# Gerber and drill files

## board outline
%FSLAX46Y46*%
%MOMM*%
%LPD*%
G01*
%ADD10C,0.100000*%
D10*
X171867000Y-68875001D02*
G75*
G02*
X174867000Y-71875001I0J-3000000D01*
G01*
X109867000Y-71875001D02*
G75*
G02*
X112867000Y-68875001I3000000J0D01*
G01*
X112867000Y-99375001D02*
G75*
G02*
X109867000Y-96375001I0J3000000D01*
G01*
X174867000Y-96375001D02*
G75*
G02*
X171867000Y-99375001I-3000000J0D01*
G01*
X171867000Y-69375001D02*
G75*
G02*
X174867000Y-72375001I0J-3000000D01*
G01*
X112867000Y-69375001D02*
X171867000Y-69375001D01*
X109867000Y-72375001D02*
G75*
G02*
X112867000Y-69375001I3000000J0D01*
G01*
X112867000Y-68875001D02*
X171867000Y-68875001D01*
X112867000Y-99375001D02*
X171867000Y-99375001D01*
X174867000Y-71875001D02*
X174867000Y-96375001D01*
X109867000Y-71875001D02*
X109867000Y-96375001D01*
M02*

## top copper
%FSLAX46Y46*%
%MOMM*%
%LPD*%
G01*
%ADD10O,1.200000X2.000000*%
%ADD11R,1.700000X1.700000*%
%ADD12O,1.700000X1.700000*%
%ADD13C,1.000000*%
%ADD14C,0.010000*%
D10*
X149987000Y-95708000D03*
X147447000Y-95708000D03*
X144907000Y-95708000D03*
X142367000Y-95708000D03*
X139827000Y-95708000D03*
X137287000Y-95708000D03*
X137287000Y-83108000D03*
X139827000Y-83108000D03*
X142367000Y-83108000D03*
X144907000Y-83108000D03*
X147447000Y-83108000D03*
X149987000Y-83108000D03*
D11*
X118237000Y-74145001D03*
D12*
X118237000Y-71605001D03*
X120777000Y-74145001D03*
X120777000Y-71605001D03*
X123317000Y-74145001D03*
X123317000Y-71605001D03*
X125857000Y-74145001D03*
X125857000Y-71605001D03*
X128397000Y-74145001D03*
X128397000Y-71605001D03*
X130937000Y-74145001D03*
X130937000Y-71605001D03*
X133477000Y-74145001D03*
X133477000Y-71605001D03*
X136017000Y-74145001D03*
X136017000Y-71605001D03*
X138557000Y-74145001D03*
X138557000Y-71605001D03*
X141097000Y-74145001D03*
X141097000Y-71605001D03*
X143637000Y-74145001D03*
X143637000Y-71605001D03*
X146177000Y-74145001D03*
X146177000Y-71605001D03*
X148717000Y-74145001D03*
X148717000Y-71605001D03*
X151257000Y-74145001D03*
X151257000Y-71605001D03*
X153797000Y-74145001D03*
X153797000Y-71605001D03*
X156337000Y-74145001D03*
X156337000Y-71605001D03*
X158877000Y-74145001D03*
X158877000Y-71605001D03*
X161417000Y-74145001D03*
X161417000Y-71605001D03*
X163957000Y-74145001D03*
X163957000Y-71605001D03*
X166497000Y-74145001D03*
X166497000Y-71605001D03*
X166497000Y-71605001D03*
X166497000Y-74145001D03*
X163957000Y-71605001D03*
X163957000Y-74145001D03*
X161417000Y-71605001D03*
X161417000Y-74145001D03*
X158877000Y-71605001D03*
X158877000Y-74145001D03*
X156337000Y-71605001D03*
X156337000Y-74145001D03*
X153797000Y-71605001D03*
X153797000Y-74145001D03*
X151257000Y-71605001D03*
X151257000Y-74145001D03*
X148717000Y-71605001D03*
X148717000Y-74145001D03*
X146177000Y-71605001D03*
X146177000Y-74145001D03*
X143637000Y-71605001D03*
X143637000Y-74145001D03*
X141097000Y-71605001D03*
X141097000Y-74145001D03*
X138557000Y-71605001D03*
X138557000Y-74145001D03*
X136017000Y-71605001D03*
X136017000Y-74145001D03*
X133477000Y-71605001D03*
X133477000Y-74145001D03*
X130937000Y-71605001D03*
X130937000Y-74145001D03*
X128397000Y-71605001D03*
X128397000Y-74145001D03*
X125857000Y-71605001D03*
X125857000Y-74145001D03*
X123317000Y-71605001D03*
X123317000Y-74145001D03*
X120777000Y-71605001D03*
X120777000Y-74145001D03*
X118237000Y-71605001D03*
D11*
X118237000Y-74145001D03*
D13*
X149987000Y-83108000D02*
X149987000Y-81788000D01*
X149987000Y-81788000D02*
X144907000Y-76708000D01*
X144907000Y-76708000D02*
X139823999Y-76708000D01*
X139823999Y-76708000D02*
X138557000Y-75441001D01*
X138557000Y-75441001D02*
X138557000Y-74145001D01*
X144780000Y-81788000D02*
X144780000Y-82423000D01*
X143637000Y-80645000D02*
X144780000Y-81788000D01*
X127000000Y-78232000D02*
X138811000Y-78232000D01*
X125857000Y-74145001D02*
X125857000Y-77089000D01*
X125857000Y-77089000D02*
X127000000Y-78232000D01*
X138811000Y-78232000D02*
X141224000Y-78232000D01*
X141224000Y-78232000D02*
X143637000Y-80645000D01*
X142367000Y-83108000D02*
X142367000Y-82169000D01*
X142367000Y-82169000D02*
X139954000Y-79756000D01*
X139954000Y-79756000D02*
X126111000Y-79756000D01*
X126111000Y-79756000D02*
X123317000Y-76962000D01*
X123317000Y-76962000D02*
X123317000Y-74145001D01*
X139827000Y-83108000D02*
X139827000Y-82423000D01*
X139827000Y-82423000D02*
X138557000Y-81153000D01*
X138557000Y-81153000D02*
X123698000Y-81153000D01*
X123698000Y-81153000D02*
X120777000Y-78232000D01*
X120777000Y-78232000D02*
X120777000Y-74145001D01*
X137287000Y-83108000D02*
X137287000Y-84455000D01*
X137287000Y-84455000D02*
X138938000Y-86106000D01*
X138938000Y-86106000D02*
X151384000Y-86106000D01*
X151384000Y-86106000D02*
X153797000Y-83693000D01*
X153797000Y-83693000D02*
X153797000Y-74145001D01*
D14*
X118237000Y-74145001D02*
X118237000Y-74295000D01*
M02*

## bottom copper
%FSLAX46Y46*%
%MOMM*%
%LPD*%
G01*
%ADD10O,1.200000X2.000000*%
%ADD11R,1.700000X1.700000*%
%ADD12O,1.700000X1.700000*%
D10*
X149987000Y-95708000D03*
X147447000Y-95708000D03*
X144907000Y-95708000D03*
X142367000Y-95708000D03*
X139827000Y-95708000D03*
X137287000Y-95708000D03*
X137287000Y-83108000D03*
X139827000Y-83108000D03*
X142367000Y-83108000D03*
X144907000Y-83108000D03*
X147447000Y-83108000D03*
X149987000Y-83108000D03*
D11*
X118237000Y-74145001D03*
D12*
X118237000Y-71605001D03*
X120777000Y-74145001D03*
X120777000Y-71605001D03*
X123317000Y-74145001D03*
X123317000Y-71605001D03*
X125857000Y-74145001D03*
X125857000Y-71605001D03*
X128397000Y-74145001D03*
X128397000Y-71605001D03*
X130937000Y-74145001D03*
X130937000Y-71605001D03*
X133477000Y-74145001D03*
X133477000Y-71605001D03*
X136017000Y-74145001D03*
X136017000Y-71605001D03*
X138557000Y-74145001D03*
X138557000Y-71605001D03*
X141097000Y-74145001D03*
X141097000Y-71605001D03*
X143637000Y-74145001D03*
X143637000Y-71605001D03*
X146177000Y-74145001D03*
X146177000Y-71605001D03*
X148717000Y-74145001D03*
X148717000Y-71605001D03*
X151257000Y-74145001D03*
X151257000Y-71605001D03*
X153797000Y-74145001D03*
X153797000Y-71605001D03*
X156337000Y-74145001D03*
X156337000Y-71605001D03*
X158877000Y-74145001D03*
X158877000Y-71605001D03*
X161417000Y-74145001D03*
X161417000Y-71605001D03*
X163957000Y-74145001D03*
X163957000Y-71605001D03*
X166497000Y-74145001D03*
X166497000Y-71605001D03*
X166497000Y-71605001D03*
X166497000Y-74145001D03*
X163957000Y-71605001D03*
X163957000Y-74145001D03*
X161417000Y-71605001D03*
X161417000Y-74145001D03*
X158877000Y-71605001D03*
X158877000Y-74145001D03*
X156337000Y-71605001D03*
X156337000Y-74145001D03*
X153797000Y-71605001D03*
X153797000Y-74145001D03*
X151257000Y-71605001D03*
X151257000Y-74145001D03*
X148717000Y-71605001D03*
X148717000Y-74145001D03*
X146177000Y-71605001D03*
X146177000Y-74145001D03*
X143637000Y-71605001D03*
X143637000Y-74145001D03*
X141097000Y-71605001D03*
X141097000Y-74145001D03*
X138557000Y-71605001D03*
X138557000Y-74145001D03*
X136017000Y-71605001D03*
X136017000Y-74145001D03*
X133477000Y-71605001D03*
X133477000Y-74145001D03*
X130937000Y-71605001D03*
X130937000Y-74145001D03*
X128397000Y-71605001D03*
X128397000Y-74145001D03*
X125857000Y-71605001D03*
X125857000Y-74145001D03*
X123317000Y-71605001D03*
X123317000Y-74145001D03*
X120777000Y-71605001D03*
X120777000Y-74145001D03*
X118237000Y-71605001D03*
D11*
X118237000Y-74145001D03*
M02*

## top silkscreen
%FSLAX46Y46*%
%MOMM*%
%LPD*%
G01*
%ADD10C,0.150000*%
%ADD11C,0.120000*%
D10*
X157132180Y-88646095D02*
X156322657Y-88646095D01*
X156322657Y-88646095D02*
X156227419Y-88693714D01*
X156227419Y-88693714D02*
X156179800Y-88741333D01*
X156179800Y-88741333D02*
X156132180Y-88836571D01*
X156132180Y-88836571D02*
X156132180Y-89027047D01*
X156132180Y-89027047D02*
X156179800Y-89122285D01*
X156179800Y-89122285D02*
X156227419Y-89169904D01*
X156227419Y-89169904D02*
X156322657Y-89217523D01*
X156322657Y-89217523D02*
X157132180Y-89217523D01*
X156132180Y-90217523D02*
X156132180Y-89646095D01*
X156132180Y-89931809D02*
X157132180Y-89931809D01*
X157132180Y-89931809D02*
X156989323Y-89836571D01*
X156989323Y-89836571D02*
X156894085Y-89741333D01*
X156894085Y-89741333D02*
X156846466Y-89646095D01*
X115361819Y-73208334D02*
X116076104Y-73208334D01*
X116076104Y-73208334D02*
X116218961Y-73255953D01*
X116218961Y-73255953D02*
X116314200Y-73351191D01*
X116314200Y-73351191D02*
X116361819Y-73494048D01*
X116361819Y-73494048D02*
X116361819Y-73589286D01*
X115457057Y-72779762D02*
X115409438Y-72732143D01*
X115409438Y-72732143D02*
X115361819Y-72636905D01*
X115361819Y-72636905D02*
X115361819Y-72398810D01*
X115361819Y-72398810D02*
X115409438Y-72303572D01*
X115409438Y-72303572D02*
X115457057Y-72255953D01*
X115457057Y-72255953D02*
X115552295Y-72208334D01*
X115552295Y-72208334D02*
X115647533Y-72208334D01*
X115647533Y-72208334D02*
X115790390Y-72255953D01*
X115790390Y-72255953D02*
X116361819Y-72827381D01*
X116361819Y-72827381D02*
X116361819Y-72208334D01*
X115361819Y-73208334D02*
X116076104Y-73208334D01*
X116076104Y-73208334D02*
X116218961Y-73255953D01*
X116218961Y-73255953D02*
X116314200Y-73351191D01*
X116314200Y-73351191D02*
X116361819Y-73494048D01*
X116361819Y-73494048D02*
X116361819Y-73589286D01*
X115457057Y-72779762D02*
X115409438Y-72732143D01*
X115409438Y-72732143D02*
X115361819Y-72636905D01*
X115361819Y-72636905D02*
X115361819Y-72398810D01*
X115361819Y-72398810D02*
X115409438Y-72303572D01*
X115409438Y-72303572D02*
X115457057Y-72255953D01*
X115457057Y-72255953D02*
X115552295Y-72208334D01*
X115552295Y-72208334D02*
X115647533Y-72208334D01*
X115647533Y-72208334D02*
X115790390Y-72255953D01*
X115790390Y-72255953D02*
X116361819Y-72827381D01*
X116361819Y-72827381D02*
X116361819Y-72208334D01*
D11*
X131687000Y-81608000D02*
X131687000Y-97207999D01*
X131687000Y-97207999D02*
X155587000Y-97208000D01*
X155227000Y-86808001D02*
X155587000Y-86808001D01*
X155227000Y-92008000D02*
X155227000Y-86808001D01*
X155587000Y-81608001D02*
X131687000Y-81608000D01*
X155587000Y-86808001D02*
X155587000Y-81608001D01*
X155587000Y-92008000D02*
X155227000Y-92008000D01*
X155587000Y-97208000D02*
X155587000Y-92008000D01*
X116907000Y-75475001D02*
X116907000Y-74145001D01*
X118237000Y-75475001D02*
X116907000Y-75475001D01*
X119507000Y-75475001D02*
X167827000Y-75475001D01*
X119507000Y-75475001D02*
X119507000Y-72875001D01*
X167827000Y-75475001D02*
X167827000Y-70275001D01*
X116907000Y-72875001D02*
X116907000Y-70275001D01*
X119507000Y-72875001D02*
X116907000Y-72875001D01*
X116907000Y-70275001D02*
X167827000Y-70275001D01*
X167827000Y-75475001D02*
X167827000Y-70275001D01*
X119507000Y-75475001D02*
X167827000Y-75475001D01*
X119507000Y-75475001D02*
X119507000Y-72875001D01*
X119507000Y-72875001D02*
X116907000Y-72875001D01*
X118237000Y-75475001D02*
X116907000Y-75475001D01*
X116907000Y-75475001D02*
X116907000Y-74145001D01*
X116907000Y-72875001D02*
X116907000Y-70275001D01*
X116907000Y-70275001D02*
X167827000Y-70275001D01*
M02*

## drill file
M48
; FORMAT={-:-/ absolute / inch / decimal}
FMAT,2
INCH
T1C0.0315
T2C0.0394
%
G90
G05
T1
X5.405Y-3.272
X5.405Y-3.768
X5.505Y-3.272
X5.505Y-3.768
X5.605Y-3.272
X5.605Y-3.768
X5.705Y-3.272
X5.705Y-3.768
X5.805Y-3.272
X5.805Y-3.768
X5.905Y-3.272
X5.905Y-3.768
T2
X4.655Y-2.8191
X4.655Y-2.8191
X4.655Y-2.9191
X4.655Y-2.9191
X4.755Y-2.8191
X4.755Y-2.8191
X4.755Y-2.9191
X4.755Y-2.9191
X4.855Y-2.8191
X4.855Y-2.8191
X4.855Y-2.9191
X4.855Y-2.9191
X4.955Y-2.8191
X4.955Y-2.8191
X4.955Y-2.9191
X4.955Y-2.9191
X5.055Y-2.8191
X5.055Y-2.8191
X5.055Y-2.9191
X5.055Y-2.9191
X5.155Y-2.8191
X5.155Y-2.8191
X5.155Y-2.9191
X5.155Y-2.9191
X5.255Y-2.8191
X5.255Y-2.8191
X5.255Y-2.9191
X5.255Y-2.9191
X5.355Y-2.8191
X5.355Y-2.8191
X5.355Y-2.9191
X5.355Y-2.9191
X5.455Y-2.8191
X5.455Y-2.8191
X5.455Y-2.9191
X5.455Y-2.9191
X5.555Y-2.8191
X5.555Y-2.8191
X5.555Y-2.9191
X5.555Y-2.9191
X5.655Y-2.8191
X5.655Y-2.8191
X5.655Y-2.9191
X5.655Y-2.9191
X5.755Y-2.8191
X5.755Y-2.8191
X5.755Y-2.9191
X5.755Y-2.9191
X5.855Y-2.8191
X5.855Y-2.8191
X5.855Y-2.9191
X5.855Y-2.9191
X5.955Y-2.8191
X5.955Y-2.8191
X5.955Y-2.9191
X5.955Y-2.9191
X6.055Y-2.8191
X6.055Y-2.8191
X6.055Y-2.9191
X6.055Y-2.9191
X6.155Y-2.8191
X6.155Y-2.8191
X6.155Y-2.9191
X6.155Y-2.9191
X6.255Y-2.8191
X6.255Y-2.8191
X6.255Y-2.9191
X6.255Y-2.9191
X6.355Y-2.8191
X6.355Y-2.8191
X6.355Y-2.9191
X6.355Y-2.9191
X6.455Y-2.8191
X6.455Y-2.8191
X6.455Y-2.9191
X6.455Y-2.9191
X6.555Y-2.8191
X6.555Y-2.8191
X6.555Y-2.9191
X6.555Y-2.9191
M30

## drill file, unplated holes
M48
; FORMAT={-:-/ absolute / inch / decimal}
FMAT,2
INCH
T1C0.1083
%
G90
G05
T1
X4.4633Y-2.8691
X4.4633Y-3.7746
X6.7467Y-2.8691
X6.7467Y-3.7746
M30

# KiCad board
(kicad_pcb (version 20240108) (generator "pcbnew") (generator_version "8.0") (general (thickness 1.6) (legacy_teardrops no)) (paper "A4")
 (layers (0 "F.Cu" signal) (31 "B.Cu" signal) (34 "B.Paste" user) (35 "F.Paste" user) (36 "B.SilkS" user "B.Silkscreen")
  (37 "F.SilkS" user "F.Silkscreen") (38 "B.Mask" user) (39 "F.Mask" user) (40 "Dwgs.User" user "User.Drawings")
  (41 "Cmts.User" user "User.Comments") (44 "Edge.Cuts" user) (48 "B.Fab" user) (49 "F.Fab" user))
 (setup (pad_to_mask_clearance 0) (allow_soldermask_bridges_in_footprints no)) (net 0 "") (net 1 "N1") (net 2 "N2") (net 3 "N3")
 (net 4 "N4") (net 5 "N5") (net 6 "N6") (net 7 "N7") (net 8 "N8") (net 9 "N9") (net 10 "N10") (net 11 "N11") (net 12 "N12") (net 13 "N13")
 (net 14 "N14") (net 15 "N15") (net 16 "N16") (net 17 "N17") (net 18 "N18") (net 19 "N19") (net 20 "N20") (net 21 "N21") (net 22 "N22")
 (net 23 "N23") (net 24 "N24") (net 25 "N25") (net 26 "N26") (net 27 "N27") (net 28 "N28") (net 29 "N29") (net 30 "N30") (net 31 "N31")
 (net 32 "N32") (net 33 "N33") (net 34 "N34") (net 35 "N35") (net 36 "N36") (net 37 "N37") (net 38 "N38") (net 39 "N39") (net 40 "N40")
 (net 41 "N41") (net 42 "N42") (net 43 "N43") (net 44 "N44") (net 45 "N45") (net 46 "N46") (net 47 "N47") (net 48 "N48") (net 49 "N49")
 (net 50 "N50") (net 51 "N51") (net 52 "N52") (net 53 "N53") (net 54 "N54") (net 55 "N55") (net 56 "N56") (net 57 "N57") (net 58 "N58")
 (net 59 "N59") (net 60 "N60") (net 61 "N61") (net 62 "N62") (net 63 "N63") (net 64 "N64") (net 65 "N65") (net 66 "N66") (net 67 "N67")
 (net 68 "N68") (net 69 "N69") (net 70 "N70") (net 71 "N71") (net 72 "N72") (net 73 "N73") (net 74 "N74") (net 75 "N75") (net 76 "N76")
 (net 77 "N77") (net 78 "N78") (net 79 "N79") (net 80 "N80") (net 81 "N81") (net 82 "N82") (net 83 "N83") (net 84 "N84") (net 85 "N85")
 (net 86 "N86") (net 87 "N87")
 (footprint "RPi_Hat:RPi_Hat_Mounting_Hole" (layer "F.Cu") (at 171.367 72.875001)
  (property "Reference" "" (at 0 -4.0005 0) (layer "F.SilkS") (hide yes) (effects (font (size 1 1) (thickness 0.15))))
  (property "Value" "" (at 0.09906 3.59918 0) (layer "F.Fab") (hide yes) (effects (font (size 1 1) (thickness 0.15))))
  (pad "" np_thru_hole circle (at 0 0) (size 2.75 2.75) (drill 2.75) (layers "*.Cu" "*.Mask") (solder_mask_margin 1.725) (clearance 1.725)))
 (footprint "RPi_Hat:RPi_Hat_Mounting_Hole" (layer "F.Cu") (at 113.367 72.875001)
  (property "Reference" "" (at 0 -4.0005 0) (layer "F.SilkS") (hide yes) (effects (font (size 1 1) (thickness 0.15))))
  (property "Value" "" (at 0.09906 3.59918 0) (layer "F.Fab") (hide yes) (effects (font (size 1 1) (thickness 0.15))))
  (pad "" np_thru_hole circle (at 0 0) (size 2.75 2.75) (drill 2.75) (layers "*.Cu" "*.Mask") (solder_mask_margin 1.725) (clearance 1.725)))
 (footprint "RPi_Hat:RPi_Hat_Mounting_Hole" (layer "F.Cu") (at 171.367 95.875001)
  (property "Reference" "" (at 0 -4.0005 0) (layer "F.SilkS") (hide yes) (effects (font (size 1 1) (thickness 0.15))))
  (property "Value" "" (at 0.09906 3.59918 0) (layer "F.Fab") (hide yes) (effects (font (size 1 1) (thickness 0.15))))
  (pad "" np_thru_hole circle (at 0 0) (size 2.75 2.75) (drill 2.75) (layers "*.Cu" "*.Mask") (solder_mask_margin 1.725) (clearance 1.725)))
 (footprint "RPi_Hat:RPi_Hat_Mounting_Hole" (layer "F.Cu") (at 113.367 95.875001)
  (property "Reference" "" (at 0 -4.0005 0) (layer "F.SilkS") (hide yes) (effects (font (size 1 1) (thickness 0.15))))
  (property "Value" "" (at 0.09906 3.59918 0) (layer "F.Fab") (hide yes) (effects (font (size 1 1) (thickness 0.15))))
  (pad "" np_thru_hole circle (at 0 0) (size 2.75 2.75) (drill 2.75) (layers "*.Cu" "*.Mask") (solder_mask_margin 1.725) (clearance 1.725)))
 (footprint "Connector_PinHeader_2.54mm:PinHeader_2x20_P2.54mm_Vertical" (layer "F.Cu") (at 118.237 74.145001 90)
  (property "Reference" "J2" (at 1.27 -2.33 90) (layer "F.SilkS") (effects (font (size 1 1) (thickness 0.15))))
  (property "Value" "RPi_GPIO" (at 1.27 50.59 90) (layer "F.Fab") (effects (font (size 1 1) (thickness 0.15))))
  (fp_line (start 3.87 -1.33) (end 3.87 49.59) (stroke (width 0.12) (type solid)) (layer "F.SilkS"))
  (fp_line (start 1.27 -1.33) (end 3.87 -1.33) (stroke (width 0.12) (type solid)) (layer "F.SilkS"))
  (fp_line (start -1.33 -1.33) (end 0 -1.33) (stroke (width 0.12) (type solid)) (layer "F.SilkS"))
  (fp_line (start -1.33 0) (end -1.33 -1.33) (stroke (width 0.12) (type solid)) (layer "F.SilkS"))
  (fp_line (start 1.27 1.27) (end 1.27 -1.33) (stroke (width 0.12) (type solid)) (layer "F.SilkS"))
  (fp_line (start -1.33 1.27) (end 1.27 1.27) (stroke (width 0.12) (type solid)) (layer "F.SilkS"))
  (fp_line (start -1.33 1.27) (end -1.33 49.59) (stroke (width 0.12) (type solid)) (layer "F.SilkS"))
  (fp_line (start -1.33 49.59) (end 3.87 49.59) (stroke (width 0.12) (type solid)) (layer "F.SilkS"))
  (pad "1" thru_hole rect (at 0 0 90) (size 1.7 1.7) (drill 1) (layers "*.Cu" "*.Mask") (remove_unused_layers no) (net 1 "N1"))
  (pad "2" thru_hole oval (at 2.54 0 90) (size 1.7 1.7) (drill 1) (layers "*.Cu" "*.Mask") (remove_unused_layers no) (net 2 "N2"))
  (pad "3" thru_hole oval (at 0 2.54 90) (size 1.7 1.7) (drill 1) (layers "*.Cu" "*.Mask") (remove_unused_layers no) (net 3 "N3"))
  (pad "4" thru_hole oval (at 2.54 2.54 90) (size 1.7 1.7) (drill 1) (layers "*.Cu" "*.Mask") (remove_unused_layers no) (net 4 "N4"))
  (pad "5" thru_hole oval (at 0 5.08 90) (size 1.7 1.7) (drill 1) (layers "*.Cu" "*.Mask") (remove_unused_layers no) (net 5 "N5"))
  (pad "6" thru_hole oval (at 2.54 5.08 90) (size 1.7 1.7) (drill 1) (layers "*.Cu" "*.Mask") (remove_unused_layers no) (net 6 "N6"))
  (pad "7" thru_hole oval (at 0 7.62 90) (size 1.7 1.7) (drill 1) (layers "*.Cu" "*.Mask") (remove_unused_layers no) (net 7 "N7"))
  (pad "8" thru_hole oval (at 2.54 7.62 90) (size 1.7 1.7) (drill 1) (layers "*.Cu" "*.Mask") (remove_unused_layers no) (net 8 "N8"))
  (pad "9" thru_hole oval (at 0 10.16 90) (size 1.7 1.7) (drill 1) (layers "*.Cu" "*.Mask") (remove_unused_layers no) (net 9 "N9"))
  (pad "10" thru_hole oval (at 2.54 10.16 90) (size 1.7 1.7) (drill 1) (layers "*.Cu" "*.Mask") (remove_unused_layers no) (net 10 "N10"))
  (pad "11" thru_hole oval (at 0 12.7 90) (size 1.7 1.7) (drill 1) (layers "*.Cu" "*.Mask") (remove_unused_layers no) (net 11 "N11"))
  (pad "12" thru_hole oval (at 2.54 12.7 90) (size 1.7 1.7) (drill 1) (layers "*.Cu" "*.Mask") (remove_unused_layers no) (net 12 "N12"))
  (pad "13" thru_hole oval (at 0 15.24 90) (size 1.7 1.7) (drill 1) (layers "*.Cu" "*.Mask") (remove_unused_layers no) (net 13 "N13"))
  (pad "14" thru_hole oval (at 2.54 15.24 90) (size 1.7 1.7) (drill 1) (layers "*.Cu" "*.Mask") (remove_unused_layers no) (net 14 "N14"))
  (pad "15" thru_hole oval (at 0 17.78 90) (size 1.7 1.7) (drill 1) (layers "*.Cu" "*.Mask") (remove_unused_layers no) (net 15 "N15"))
  (pad "16" thru_hole oval (at 2.54 17.78 90) (size 1.7 1.7) (drill 1) (layers "*.Cu" "*.Mask") (remove_unused_layers no) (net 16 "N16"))
  (pad "17" thru_hole oval (at 0 20.32 90) (size 1.7 1.7) (drill 1) (layers "*.Cu" "*.Mask") (remove_unused_layers no) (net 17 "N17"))
  (pad "18" thru_hole oval (at 2.54 20.32 90) (size 1.7 1.7) (drill 1) (layers "*.Cu" "*.Mask") (remove_unused_layers no) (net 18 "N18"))
  (pad "19" thru_hole oval (at 0 22.86 90) (size 1.7 1.7) (drill 1) (layers "*.Cu" "*.Mask") (remove_unused_layers no) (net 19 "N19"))
  (pad "20" thru_hole oval (at 2.54 22.86 90) (size 1.7 1.7) (drill 1) (layers "*.Cu" "*.Mask") (remove_unused_layers no) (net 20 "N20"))
  (pad "21" thru_hole oval (at 0 25.4 90) (size 1.7 1.7) (drill 1) (layers "*.Cu" "*.Mask") (remove_unused_layers no) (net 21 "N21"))
  (pad "22" thru_hole oval (at 2.54 25.4 90) (size 1.7 1.7) (drill 1) (layers "*.Cu" "*.Mask") (remove_unused_layers no) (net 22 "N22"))
  (pad "23" thru_hole oval (at 0 27.94 90) (size 1.7 1.7) (drill 1) (layers "*.Cu" "*.Mask") (remove_unused_layers no) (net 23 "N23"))
  (pad "24" thru_hole oval (at 2.54 27.94 90) (size 1.7 1.7) (drill 1) (layers "*.Cu" "*.Mask") (remove_unused_layers no) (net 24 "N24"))
  (pad "25" thru_hole oval (at 0 30.48 90) (size 1.7 1.7) (drill 1) (layers "*.Cu" "*.Mask") (remove_unused_layers no) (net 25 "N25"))
  (pad "26" thru_hole oval (at 2.54 30.48 90) (size 1.7 1.7) (drill 1) (layers "*.Cu" "*.Mask") (remove_unused_layers no) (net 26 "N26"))
  (pad "27" thru_hole oval (at 0 33.02 90) (size 1.7 1.7) (drill 1) (layers "*.Cu" "*.Mask") (remove_unused_layers no) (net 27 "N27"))
  (pad "28" thru_hole oval (at 2.54 33.02 90) (size 1.7 1.7) (drill 1) (layers "*.Cu" "*.Mask") (remove_unused_layers no) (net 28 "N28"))
  (pad "29" thru_hole oval (at 0 35.56 90) (size 1.7 1.7) (drill 1) (layers "*.Cu" "*.Mask") (remove_unused_layers no) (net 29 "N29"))
  (pad "30" thru_hole oval (at 2.54 35.56 90) (size 1.7 1.7) (drill 1) (layers "*.Cu" "*.Mask") (remove_unused_layers no) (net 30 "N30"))
  (pad "31" thru_hole oval (at 0 38.1 90) (size 1.7 1.7) (drill 1) (layers "*.Cu" "*.Mask") (remove_unused_layers no) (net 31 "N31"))
  (pad "32" thru_hole oval (at 2.54 38.1 90) (size 1.7 1.7) (drill 1) (layers "*.Cu" "*.Mask") (remove_unused_layers no) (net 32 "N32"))
  (pad "33" thru_hole oval (at 0 40.64 90) (size 1.7 1.7) (drill 1) (layers "*.Cu" "*.Mask") (remove_unused_layers no) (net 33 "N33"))
  (pad "34" thru_hole oval (at 2.54 40.64 90) (size 1.7 1.7) (drill 1) (layers "*.Cu" "*.Mask") (remove_unused_layers no) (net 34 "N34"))
  (pad "35" thru_hole oval (at 0 43.18 90) (size 1.7 1.7) (drill 1) (layers "*.Cu" "*.Mask") (remove_unused_layers no) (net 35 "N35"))
  (pad "36" thru_hole oval (at 2.54 43.18 90) (size 1.7 1.7) (drill 1) (layers "*.Cu" "*.Mask") (remove_unused_layers no) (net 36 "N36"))
  (pad "37" thru_hole oval (at 0 45.72 90) (size 1.7 1.7) (drill 1) (layers "*.Cu" "*.Mask") (remove_unused_layers no) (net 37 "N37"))
  (pad "38" thru_hole oval (at 2.54 45.72 90) (size 1.7 1.7) (drill 1) (layers "*.Cu" "*.Mask") (remove_unused_layers no) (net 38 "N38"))
  (pad "39" thru_hole oval (at 0 48.26 90) (size 1.7 1.7) (drill 1) (layers "*.Cu" "*.Mask") (remove_unused_layers no) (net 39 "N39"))
  (pad "40" thru_hole oval (at 2.54 48.26 90) (size 1.7 1.7) (drill 1) (layers "*.Cu" "*.Mask") (remove_unused_layers no) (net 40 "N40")))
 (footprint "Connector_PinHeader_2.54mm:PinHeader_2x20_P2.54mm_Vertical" (layer "F.Cu") (at 118.237 74.145001 90)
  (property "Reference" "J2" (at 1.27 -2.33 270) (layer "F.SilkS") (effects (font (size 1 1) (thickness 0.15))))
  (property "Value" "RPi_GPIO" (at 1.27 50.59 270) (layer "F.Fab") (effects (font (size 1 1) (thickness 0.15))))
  (fp_line (start 3.87 -1.33) (end 3.87 49.59) (stroke (width 0.12) (type solid)) (layer "F.SilkS"))
  (fp_line (start 1.27 -1.33) (end 3.87 -1.33) (stroke (width 0.12) (type solid)) (layer "F.SilkS"))
  (fp_line (start -1.33 -1.33) (end 0 -1.33) (stroke (width 0.12) (type solid)) (layer "F.SilkS"))
  (fp_line (start -1.33 0) (end -1.33 -1.33) (stroke (width 0.12) (type solid)) (layer "F.SilkS"))
  (fp_line (start 1.27 1.27) (end 1.27 -1.33) (stroke (width 0.12) (type solid)) (layer "F.SilkS"))
  (fp_line (start -1.33 1.27) (end 1.27 1.27) (stroke (width 0.12) (type solid)) (layer "F.SilkS"))
  (fp_line (start -1.33 1.27) (end -1.33 49.59) (stroke (width 0.12) (type solid)) (layer "F.SilkS"))
  (fp_line (start -1.33 49.59) (end 3.87 49.59) (stroke (width 0.12) (type solid)) (layer "F.SilkS"))
  (pad "1" thru_hole rect (at 0 0 90) (size 1.7 1.7) (drill 1) (layers "*.Cu" "*.Mask") (remove_unused_layers no) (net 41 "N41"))
  (pad "2" thru_hole oval (at 2.54 0 90) (size 1.7 1.7) (drill 1) (layers "*.Cu" "*.Mask") (remove_unused_layers no) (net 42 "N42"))
  (pad "3" thru_hole oval (at 0 2.54 90) (size 1.7 1.7) (drill 1) (layers "*.Cu" "*.Mask") (remove_unused_layers no) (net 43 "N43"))
  (pad "4" thru_hole oval (at 2.54 2.54 90) (size 1.7 1.7) (drill 1) (layers "*.Cu" "*.Mask") (remove_unused_layers no) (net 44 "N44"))
  (pad "5" thru_hole oval (at 0 5.08 90) (size 1.7 1.7) (drill 1) (layers "*.Cu" "*.Mask") (remove_unused_layers no) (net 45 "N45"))
  (pad "6" thru_hole oval (at 2.54 5.08 90) (size 1.7 1.7) (drill 1) (layers "*.Cu" "*.Mask") (remove_unused_layers no) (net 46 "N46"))
  (pad "7" thru_hole oval (at 0 7.62 90) (size 1.7 1.7) (drill 1) (layers "*.Cu" "*.Mask") (remove_unused_layers no) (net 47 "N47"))
  (pad "8" thru_hole oval (at 2.54 7.62 90) (size 1.7 1.7) (drill 1) (layers "*.Cu" "*.Mask") (remove_unused_layers no) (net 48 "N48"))
  (pad "9" thru_hole oval (at 0 10.16 90) (size 1.7 1.7) (drill 1) (layers "*.Cu" "*.Mask") (remove_unused_layers no) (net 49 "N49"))
  (pad "10" thru_hole oval (at 2.54 10.16 90) (size 1.7 1.7) (drill 1) (layers "*.Cu" "*.Mask") (remove_unused_layers no) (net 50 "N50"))
  (pad "11" thru_hole oval (at 0 12.7 90) (size 1.7 1.7) (drill 1) (layers "*.Cu" "*.Mask") (remove_unused_layers no) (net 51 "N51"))
  (pad "12" thru_hole oval (at 2.54 12.7 90) (size 1.7 1.7) (drill 1) (layers "*.Cu" "*.Mask") (remove_unused_layers no) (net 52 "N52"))
  (pad "13" thru_hole oval (at 0 15.24 90) (size 1.7 1.7) (drill 1) (layers "*.Cu" "*.Mask") (remove_unused_layers no) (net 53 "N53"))
  (pad "14" thru_hole oval (at 2.54 15.24 90) (size 1.7 1.7) (drill 1) (layers "*.Cu" "*.Mask") (remove_unused_layers no) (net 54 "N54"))
  (pad "15" thru_hole oval (at 0 17.78 90) (size 1.7 1.7) (drill 1) (layers "*.Cu" "*.Mask") (remove_unused_layers no) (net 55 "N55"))
  (pad "16" thru_hole oval (at 2.54 17.78 90) (size 1.7 1.7) (drill 1) (layers "*.Cu" "*.Mask") (remove_unused_layers no) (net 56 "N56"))
  (pad "17" thru_hole oval (at 0 20.32 90) (size 1.7 1.7) (drill 1) (layers "*.Cu" "*.Mask") (remove_unused_layers no) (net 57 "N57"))
  (pad "18" thru_hole oval (at 2.54 20.32 90) (size 1.7 1.7) (drill 1) (layers "*.Cu" "*.Mask") (remove_unused_layers no) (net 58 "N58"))
  (pad "19" thru_hole oval (at 0 22.86 90) (size 1.7 1.7) (drill 1) (layers "*.Cu" "*.Mask") (remove_unused_layers no) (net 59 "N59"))
  (pad "20" thru_hole oval (at 2.54 22.86 90) (size 1.7 1.7) (drill 1) (layers "*.Cu" "*.Mask") (remove_unused_layers no) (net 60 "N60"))
  (pad "21" thru_hole oval (at 0 25.4 90) (size 1.7 1.7) (drill 1) (layers "*.Cu" "*.Mask") (remove_unused_layers no) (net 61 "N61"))
  (pad "22" thru_hole oval (at 2.54 25.4 90) (size 1.7 1.7) (drill 1) (layers "*.Cu" "*.Mask") (remove_unused_layers no) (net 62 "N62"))
  (pad "23" thru_hole oval (at 0 27.94 90) (size 1.7 1.7) (drill 1) (layers "*.Cu" "*.Mask") (remove_unused_layers no) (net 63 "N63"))
  (pad "24" thru_hole oval (at 2.54 27.94 90) (size 1.7 1.7) (drill 1) (layers "*.Cu" "*.Mask") (remove_unused_layers no) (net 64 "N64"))
  (pad "25" thru_hole oval (at 0 30.48 90) (size 1.7 1.7) (drill 1) (layers "*.Cu" "*.Mask") (remove_unused_layers no) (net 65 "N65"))
  (pad "26" thru_hole oval (at 2.54 30.48 90) (size 1.7 1.7) (drill 1) (layers "*.Cu" "*.Mask") (remove_unused_layers no) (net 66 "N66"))
  (pad "27" thru_hole oval (at 0 33.02 90) (size 1.7 1.7) (drill 1) (layers "*.Cu" "*.Mask") (remove_unused_layers no) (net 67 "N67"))
  (pad "28" thru_hole oval (at 2.54 33.02 90) (size 1.7 1.7) (drill 1) (layers "*.Cu" "*.Mask") (remove_unused_layers no) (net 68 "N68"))
  (pad "29" thru_hole oval (at 0 35.56 90) (size 1.7 1.7) (drill 1) (layers "*.Cu" "*.Mask") (remove_unused_layers no) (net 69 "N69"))
  (pad "30" thru_hole oval (at 2.54 35.56 90) (size 1.7 1.7) (drill 1) (layers "*.Cu" "*.Mask") (remove_unused_layers no) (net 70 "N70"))
  (pad "31" thru_hole oval (at 0 38.1 90) (size 1.7 1.7) (drill 1) (layers "*.Cu" "*.Mask") (remove_unused_layers no) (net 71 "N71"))
  (pad "32" thru_hole oval (at 2.54 38.1 90) (size 1.7 1.7) (drill 1) (layers "*.Cu" "*.Mask") (remove_unused_layers no) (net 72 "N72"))
  (pad "33" thru_hole oval (at 0 40.64 90) (size 1.7 1.7) (drill 1) (layers "*.Cu" "*.Mask") (remove_unused_layers no) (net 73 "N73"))
  (pad "34" thru_hole oval (at 2.54 40.64 90) (size 1.7 1.7) (drill 1) (layers "*.Cu" "*.Mask") (remove_unused_layers no) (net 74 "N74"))
  (pad "35" thru_hole oval (at 0 43.18 90) (size 1.7 1.7) (drill 1) (layers "*.Cu" "*.Mask") (remove_unused_layers no) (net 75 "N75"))
  (pad "36" thru_hole oval (at 2.54 43.18 90) (size 1.7 1.7) (drill 1) (layers "*.Cu" "*.Mask") (remove_unused_layers no) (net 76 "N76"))
  (pad "37" thru_hole oval (at 0 45.72 90) (size 1.7 1.7) (drill 1) (layers "*.Cu" "*.Mask") (remove_unused_layers no) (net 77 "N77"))
  (pad "38" thru_hole oval (at 2.54 45.72 90) (size 1.7 1.7) (drill 1) (layers "*.Cu" "*.Mask") (remove_unused_layers no) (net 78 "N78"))
  (pad "39" thru_hole oval (at 0 48.26 90) (size 1.7 1.7) (drill 1) (layers "*.Cu" "*.Mask") (remove_unused_layers no) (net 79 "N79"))
  (pad "40" thru_hole oval (at 2.54 48.26 90) (size 1.7 1.7) (drill 1) (layers "*.Cu" "*.Mask") (remove_unused_layers no) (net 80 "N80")))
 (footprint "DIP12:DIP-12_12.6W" (layer "F.Cu") (at 143.637 89.408 180)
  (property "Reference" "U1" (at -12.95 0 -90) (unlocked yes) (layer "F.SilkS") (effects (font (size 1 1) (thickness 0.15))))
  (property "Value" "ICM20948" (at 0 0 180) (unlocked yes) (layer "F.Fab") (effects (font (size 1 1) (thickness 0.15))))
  (fp_line (start 11.95 7.8) (end 11.95 -7.799999) (stroke (width 0.12) (type default)) (layer "F.SilkS"))
  (fp_line (start 11.95 -7.799999) (end -11.95 -7.8) (stroke (width 0.12) (type default)) (layer "F.SilkS"))
  (fp_line (start -11.59 2.599999) (end -11.95 2.599999) (stroke (width 0.12) (type default)) (layer "F.SilkS"))
  (fp_line (start -11.59 -2.6) (end -11.59 2.599999) (stroke (width 0.12) (type default)) (layer "F.SilkS"))
  (fp_line (start -11.95 7.799999) (end 11.95 7.8) (stroke (width 0.12) (type default)) (layer "F.SilkS"))
  (fp_line (start -11.95 2.599999) (end -11.95 7.799999) (stroke (width 0.12) (type default)) (layer "F.SilkS"))
  (fp_line (start -11.95 -2.6) (end -11.59 -2.6) (stroke (width 0.12) (type default)) (layer "F.SilkS"))
  (fp_line (start -11.95 -7.8) (end -11.95 -2.6) (stroke (width 0.12) (type default)) (layer "F.SilkS"))
  (pad "1" thru_hole oval (at -6.35 6.3 180) (size 1.2 2) (drill 0.8) (layers "*.Cu" "*.Mask") (remove_unused_layers no) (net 57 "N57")
   (thermal_bridge_angle 45))
  (pad "2" thru_hole oval (at -3.81 6.3 180) (size 1.2 2) (drill 0.8) (layers "*.Cu" "*.Mask") (remove_unused_layers no) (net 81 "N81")
   (thermal_bridge_angle 45))
  (pad "3" thru_hole oval (at -1.27 6.3 180) (size 1.2 2) (drill 0.8) (layers "*.Cu" "*.Mask") (remove_unused_layers no) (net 49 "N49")
   (thermal_bridge_angle 45))
  (pad "4" thru_hole oval (at 1.27 6.3 180) (size 1.2 2) (drill 0.8) (layers "*.Cu" "*.Mask") (remove_unused_layers no) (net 45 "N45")
   (thermal_bridge_angle 45))
  (pad "5" thru_hole oval (at 3.81 6.3 180) (size 1.2 2) (drill 0.8) (layers "*.Cu" "*.Mask") (remove_unused_layers no) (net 43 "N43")
   (thermal_bridge_angle 45))
  (pad "6" thru_hole oval (at 6.35 6.3 180) (size 1.2 2) (drill 0.8) (layers "*.Cu" "*.Mask") (remove_unused_layers no) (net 69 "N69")
   (thermal_bridge_angle 45))
  (pad "7" thru_hole oval (at 6.35 -6.3 180) (size 1.2 2) (drill 0.8) (layers "*.Cu" "*.Mask") (remove_unused_layers no) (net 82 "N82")
   (thermal_bridge_angle 45))
  (pad "8" thru_hole oval (at 3.81 -6.3 180) (size 1.2 2) (drill 0.8) (layers "*.Cu" "*.Mask") (remove_unused_layers no) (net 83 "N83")
   (thermal_bridge_angle 45))
  (pad "9" thru_hole oval (at 1.27 -6.3 180) (size 1.2 2) (drill 0.8) (layers "*.Cu" "*.Mask") (remove_unused_layers no) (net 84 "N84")
   (thermal_bridge_angle 45))
  (pad "10" thru_hole oval (at -1.27 -6.3 180) (size 1.2 2) (drill 0.8) (layers "*.Cu" "*.Mask") (remove_unused_layers no) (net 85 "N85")
   (thermal_bridge_angle 45))
  (pad "11" thru_hole oval (at -3.81 -6.3 180) (size 1.2 2) (drill 0.8) (layers "*.Cu" "*.Mask") (remove_unused_layers no) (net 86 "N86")
   (thermal_bridge_angle 45))
  (pad "12" thru_hole oval (at -6.35 -6.3 180) (size 1.2 2) (drill 0.8) (layers "*.Cu" "*.Mask") (remove_unused_layers no) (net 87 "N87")
   (thermal_bridge_angle 45)))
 (gr_arc (start 171.867 68.875001) (mid 173.98832 69.753681) (end 174.867 71.875001) (stroke (width 0.1) (type solid)) (layer "Edge.Cuts"))
 (gr_arc (start 109.867 71.875001) (mid 110.74568 69.753681) (end 112.867 68.875001) (stroke (width 0.1) (type solid)) (layer "Edge.Cuts"))
 (gr_arc (start 112.867 99.375001) (mid 110.74568 98.496321) (end 109.867 96.375001) (stroke (width 0.1) (type solid)) (layer "Edge.Cuts"))
 (gr_arc (start 174.867 96.375001) (mid 173.98832 98.496321) (end 171.867 99.375001) (stroke (width 0.1) (type solid)) (layer "Edge.Cuts"))
 (gr_arc (start 171.867 69.375001) (mid 173.98832 70.253681) (end 174.867 72.375001) (stroke (width 0.1) (type solid)) (layer "Edge.Cuts"))
 (gr_line (start 112.867 69.375001) (end 171.867 69.375001) (stroke (width 0.1) (type solid)) (layer "Edge.Cuts"))
 (gr_arc (start 109.867 72.375001) (mid 110.74568 70.253681) (end 112.867 69.375001) (stroke (width 0.1) (type solid)) (layer "Edge.Cuts"))
 (gr_line (start 112.867 68.875001) (end 171.867 68.875001) (stroke (width 0.1) (type solid)) (layer "Edge.Cuts"))
 (gr_line (start 112.867 99.375001) (end 171.867 99.375001) (stroke (width 0.1) (type solid)) (layer "Edge.Cuts"))
 (gr_line (start 174.867 71.875001) (end 174.867 96.375001) (stroke (width 0.1) (type solid)) (layer "Edge.Cuts"))
 (gr_line (start 109.867 71.875001) (end 109.867 96.375001) (stroke (width 0.1) (type solid)) (layer "Edge.Cuts"))
 (segment (start 118.237 74.145001) (end 118.237 74.295) (width 0.01) (layer "F.Cu") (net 1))
 (segment (start 141.224 78.232) (end 143.637 80.645) (width 1) (layer "F.Cu") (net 47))
 (segment (start 125.857 74.145001) (end 125.857 77.089) (width 1) (layer "F.Cu") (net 47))
 (segment (start 138.811 78.232) (end 141.224 78.232) (width 1) (layer "F.Cu") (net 47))
 (segment (start 144.78 81.788) (end 144.78 82.423) (width 1) (layer "F.Cu") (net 47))
 (segment (start 127 78.232) (end 138.811 78.232) (width 1) (layer "F.Cu") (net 47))
 (segment (start 125.857 77.089) (end 127 78.232) (width 1) (layer "F.Cu") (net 47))
 (segment (start 143.637 80.645) (end 144.78 81.788) (width 1) (layer "F.Cu") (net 47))
 (segment (start 123.698 81.153) (end 120.777 78.232) (width 1) (layer "F.Cu") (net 43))
 (segment (start 139.827 83.108) (end 139.827 82.423) (width 1) (layer "F.Cu") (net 43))
 (segment (start 120.777 78.232) (end 120.777 74.145001) (width 1) (layer "F.Cu") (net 43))
 (segment (start 139.827 82.423) (end 138.557 81.153) (width 1) (layer "F.Cu") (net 43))
 (segment (start 138.557 81.153) (end 123.698 81.153) (width 1) (layer "F.Cu") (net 43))
 (segment (start 139.823999 76.708) (end 138.557 75.441001) (width 1) (layer "F.Cu") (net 57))
 (segment (start 144.907 76.708) (end 139.823999 76.708) (width 1) (layer "F.Cu") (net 57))
 (segment (start 149.987 83.108) (end 149.987 81.788) (width 1) (layer "F.Cu") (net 57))
 (segment (start 149.987 81.788) (end 144.907 76.708) (width 1) (layer "F.Cu") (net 57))
 (segment (start 138.557 75.441001) (end 138.557 74.145001) (width 1) (layer "F.Cu") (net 57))
 (segment (start 139.954 79.756) (end 126.111 79.756) (width 1) (layer "F.Cu") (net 45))
 (segment (start 142.367 83.108) (end 142.367 82.169) (width 1) (layer "F.Cu") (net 45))
 (segment (start 123.317 76.962) (end 123.317 74.145001) (width 1) (layer "F.Cu") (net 45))
 (segment (start 142.367 82.169) (end 139.954 79.756) (width 1) (layer "F.Cu") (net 45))
 (segment (start 126.111 79.756) (end 123.317 76.962) (width 1) (layer "F.Cu") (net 45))
 (segment (start 137.287 84.455) (end 138.938 86.106) (width 1) (layer "F.Cu") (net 69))
 (segment (start 138.938 86.106) (end 151.384 86.106) (width 1) (layer "F.Cu") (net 69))
 (segment (start 153.797 83.693) (end 153.797 74.145001) (width 1) (layer "F.Cu") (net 69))
 (segment (start 137.287 83.108) (end 137.287 84.455) (width 1) (layer "F.Cu") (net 69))
 (segment (start 151.384 86.106) (end 153.797 83.693) (width 1) (layer "F.Cu") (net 69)))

